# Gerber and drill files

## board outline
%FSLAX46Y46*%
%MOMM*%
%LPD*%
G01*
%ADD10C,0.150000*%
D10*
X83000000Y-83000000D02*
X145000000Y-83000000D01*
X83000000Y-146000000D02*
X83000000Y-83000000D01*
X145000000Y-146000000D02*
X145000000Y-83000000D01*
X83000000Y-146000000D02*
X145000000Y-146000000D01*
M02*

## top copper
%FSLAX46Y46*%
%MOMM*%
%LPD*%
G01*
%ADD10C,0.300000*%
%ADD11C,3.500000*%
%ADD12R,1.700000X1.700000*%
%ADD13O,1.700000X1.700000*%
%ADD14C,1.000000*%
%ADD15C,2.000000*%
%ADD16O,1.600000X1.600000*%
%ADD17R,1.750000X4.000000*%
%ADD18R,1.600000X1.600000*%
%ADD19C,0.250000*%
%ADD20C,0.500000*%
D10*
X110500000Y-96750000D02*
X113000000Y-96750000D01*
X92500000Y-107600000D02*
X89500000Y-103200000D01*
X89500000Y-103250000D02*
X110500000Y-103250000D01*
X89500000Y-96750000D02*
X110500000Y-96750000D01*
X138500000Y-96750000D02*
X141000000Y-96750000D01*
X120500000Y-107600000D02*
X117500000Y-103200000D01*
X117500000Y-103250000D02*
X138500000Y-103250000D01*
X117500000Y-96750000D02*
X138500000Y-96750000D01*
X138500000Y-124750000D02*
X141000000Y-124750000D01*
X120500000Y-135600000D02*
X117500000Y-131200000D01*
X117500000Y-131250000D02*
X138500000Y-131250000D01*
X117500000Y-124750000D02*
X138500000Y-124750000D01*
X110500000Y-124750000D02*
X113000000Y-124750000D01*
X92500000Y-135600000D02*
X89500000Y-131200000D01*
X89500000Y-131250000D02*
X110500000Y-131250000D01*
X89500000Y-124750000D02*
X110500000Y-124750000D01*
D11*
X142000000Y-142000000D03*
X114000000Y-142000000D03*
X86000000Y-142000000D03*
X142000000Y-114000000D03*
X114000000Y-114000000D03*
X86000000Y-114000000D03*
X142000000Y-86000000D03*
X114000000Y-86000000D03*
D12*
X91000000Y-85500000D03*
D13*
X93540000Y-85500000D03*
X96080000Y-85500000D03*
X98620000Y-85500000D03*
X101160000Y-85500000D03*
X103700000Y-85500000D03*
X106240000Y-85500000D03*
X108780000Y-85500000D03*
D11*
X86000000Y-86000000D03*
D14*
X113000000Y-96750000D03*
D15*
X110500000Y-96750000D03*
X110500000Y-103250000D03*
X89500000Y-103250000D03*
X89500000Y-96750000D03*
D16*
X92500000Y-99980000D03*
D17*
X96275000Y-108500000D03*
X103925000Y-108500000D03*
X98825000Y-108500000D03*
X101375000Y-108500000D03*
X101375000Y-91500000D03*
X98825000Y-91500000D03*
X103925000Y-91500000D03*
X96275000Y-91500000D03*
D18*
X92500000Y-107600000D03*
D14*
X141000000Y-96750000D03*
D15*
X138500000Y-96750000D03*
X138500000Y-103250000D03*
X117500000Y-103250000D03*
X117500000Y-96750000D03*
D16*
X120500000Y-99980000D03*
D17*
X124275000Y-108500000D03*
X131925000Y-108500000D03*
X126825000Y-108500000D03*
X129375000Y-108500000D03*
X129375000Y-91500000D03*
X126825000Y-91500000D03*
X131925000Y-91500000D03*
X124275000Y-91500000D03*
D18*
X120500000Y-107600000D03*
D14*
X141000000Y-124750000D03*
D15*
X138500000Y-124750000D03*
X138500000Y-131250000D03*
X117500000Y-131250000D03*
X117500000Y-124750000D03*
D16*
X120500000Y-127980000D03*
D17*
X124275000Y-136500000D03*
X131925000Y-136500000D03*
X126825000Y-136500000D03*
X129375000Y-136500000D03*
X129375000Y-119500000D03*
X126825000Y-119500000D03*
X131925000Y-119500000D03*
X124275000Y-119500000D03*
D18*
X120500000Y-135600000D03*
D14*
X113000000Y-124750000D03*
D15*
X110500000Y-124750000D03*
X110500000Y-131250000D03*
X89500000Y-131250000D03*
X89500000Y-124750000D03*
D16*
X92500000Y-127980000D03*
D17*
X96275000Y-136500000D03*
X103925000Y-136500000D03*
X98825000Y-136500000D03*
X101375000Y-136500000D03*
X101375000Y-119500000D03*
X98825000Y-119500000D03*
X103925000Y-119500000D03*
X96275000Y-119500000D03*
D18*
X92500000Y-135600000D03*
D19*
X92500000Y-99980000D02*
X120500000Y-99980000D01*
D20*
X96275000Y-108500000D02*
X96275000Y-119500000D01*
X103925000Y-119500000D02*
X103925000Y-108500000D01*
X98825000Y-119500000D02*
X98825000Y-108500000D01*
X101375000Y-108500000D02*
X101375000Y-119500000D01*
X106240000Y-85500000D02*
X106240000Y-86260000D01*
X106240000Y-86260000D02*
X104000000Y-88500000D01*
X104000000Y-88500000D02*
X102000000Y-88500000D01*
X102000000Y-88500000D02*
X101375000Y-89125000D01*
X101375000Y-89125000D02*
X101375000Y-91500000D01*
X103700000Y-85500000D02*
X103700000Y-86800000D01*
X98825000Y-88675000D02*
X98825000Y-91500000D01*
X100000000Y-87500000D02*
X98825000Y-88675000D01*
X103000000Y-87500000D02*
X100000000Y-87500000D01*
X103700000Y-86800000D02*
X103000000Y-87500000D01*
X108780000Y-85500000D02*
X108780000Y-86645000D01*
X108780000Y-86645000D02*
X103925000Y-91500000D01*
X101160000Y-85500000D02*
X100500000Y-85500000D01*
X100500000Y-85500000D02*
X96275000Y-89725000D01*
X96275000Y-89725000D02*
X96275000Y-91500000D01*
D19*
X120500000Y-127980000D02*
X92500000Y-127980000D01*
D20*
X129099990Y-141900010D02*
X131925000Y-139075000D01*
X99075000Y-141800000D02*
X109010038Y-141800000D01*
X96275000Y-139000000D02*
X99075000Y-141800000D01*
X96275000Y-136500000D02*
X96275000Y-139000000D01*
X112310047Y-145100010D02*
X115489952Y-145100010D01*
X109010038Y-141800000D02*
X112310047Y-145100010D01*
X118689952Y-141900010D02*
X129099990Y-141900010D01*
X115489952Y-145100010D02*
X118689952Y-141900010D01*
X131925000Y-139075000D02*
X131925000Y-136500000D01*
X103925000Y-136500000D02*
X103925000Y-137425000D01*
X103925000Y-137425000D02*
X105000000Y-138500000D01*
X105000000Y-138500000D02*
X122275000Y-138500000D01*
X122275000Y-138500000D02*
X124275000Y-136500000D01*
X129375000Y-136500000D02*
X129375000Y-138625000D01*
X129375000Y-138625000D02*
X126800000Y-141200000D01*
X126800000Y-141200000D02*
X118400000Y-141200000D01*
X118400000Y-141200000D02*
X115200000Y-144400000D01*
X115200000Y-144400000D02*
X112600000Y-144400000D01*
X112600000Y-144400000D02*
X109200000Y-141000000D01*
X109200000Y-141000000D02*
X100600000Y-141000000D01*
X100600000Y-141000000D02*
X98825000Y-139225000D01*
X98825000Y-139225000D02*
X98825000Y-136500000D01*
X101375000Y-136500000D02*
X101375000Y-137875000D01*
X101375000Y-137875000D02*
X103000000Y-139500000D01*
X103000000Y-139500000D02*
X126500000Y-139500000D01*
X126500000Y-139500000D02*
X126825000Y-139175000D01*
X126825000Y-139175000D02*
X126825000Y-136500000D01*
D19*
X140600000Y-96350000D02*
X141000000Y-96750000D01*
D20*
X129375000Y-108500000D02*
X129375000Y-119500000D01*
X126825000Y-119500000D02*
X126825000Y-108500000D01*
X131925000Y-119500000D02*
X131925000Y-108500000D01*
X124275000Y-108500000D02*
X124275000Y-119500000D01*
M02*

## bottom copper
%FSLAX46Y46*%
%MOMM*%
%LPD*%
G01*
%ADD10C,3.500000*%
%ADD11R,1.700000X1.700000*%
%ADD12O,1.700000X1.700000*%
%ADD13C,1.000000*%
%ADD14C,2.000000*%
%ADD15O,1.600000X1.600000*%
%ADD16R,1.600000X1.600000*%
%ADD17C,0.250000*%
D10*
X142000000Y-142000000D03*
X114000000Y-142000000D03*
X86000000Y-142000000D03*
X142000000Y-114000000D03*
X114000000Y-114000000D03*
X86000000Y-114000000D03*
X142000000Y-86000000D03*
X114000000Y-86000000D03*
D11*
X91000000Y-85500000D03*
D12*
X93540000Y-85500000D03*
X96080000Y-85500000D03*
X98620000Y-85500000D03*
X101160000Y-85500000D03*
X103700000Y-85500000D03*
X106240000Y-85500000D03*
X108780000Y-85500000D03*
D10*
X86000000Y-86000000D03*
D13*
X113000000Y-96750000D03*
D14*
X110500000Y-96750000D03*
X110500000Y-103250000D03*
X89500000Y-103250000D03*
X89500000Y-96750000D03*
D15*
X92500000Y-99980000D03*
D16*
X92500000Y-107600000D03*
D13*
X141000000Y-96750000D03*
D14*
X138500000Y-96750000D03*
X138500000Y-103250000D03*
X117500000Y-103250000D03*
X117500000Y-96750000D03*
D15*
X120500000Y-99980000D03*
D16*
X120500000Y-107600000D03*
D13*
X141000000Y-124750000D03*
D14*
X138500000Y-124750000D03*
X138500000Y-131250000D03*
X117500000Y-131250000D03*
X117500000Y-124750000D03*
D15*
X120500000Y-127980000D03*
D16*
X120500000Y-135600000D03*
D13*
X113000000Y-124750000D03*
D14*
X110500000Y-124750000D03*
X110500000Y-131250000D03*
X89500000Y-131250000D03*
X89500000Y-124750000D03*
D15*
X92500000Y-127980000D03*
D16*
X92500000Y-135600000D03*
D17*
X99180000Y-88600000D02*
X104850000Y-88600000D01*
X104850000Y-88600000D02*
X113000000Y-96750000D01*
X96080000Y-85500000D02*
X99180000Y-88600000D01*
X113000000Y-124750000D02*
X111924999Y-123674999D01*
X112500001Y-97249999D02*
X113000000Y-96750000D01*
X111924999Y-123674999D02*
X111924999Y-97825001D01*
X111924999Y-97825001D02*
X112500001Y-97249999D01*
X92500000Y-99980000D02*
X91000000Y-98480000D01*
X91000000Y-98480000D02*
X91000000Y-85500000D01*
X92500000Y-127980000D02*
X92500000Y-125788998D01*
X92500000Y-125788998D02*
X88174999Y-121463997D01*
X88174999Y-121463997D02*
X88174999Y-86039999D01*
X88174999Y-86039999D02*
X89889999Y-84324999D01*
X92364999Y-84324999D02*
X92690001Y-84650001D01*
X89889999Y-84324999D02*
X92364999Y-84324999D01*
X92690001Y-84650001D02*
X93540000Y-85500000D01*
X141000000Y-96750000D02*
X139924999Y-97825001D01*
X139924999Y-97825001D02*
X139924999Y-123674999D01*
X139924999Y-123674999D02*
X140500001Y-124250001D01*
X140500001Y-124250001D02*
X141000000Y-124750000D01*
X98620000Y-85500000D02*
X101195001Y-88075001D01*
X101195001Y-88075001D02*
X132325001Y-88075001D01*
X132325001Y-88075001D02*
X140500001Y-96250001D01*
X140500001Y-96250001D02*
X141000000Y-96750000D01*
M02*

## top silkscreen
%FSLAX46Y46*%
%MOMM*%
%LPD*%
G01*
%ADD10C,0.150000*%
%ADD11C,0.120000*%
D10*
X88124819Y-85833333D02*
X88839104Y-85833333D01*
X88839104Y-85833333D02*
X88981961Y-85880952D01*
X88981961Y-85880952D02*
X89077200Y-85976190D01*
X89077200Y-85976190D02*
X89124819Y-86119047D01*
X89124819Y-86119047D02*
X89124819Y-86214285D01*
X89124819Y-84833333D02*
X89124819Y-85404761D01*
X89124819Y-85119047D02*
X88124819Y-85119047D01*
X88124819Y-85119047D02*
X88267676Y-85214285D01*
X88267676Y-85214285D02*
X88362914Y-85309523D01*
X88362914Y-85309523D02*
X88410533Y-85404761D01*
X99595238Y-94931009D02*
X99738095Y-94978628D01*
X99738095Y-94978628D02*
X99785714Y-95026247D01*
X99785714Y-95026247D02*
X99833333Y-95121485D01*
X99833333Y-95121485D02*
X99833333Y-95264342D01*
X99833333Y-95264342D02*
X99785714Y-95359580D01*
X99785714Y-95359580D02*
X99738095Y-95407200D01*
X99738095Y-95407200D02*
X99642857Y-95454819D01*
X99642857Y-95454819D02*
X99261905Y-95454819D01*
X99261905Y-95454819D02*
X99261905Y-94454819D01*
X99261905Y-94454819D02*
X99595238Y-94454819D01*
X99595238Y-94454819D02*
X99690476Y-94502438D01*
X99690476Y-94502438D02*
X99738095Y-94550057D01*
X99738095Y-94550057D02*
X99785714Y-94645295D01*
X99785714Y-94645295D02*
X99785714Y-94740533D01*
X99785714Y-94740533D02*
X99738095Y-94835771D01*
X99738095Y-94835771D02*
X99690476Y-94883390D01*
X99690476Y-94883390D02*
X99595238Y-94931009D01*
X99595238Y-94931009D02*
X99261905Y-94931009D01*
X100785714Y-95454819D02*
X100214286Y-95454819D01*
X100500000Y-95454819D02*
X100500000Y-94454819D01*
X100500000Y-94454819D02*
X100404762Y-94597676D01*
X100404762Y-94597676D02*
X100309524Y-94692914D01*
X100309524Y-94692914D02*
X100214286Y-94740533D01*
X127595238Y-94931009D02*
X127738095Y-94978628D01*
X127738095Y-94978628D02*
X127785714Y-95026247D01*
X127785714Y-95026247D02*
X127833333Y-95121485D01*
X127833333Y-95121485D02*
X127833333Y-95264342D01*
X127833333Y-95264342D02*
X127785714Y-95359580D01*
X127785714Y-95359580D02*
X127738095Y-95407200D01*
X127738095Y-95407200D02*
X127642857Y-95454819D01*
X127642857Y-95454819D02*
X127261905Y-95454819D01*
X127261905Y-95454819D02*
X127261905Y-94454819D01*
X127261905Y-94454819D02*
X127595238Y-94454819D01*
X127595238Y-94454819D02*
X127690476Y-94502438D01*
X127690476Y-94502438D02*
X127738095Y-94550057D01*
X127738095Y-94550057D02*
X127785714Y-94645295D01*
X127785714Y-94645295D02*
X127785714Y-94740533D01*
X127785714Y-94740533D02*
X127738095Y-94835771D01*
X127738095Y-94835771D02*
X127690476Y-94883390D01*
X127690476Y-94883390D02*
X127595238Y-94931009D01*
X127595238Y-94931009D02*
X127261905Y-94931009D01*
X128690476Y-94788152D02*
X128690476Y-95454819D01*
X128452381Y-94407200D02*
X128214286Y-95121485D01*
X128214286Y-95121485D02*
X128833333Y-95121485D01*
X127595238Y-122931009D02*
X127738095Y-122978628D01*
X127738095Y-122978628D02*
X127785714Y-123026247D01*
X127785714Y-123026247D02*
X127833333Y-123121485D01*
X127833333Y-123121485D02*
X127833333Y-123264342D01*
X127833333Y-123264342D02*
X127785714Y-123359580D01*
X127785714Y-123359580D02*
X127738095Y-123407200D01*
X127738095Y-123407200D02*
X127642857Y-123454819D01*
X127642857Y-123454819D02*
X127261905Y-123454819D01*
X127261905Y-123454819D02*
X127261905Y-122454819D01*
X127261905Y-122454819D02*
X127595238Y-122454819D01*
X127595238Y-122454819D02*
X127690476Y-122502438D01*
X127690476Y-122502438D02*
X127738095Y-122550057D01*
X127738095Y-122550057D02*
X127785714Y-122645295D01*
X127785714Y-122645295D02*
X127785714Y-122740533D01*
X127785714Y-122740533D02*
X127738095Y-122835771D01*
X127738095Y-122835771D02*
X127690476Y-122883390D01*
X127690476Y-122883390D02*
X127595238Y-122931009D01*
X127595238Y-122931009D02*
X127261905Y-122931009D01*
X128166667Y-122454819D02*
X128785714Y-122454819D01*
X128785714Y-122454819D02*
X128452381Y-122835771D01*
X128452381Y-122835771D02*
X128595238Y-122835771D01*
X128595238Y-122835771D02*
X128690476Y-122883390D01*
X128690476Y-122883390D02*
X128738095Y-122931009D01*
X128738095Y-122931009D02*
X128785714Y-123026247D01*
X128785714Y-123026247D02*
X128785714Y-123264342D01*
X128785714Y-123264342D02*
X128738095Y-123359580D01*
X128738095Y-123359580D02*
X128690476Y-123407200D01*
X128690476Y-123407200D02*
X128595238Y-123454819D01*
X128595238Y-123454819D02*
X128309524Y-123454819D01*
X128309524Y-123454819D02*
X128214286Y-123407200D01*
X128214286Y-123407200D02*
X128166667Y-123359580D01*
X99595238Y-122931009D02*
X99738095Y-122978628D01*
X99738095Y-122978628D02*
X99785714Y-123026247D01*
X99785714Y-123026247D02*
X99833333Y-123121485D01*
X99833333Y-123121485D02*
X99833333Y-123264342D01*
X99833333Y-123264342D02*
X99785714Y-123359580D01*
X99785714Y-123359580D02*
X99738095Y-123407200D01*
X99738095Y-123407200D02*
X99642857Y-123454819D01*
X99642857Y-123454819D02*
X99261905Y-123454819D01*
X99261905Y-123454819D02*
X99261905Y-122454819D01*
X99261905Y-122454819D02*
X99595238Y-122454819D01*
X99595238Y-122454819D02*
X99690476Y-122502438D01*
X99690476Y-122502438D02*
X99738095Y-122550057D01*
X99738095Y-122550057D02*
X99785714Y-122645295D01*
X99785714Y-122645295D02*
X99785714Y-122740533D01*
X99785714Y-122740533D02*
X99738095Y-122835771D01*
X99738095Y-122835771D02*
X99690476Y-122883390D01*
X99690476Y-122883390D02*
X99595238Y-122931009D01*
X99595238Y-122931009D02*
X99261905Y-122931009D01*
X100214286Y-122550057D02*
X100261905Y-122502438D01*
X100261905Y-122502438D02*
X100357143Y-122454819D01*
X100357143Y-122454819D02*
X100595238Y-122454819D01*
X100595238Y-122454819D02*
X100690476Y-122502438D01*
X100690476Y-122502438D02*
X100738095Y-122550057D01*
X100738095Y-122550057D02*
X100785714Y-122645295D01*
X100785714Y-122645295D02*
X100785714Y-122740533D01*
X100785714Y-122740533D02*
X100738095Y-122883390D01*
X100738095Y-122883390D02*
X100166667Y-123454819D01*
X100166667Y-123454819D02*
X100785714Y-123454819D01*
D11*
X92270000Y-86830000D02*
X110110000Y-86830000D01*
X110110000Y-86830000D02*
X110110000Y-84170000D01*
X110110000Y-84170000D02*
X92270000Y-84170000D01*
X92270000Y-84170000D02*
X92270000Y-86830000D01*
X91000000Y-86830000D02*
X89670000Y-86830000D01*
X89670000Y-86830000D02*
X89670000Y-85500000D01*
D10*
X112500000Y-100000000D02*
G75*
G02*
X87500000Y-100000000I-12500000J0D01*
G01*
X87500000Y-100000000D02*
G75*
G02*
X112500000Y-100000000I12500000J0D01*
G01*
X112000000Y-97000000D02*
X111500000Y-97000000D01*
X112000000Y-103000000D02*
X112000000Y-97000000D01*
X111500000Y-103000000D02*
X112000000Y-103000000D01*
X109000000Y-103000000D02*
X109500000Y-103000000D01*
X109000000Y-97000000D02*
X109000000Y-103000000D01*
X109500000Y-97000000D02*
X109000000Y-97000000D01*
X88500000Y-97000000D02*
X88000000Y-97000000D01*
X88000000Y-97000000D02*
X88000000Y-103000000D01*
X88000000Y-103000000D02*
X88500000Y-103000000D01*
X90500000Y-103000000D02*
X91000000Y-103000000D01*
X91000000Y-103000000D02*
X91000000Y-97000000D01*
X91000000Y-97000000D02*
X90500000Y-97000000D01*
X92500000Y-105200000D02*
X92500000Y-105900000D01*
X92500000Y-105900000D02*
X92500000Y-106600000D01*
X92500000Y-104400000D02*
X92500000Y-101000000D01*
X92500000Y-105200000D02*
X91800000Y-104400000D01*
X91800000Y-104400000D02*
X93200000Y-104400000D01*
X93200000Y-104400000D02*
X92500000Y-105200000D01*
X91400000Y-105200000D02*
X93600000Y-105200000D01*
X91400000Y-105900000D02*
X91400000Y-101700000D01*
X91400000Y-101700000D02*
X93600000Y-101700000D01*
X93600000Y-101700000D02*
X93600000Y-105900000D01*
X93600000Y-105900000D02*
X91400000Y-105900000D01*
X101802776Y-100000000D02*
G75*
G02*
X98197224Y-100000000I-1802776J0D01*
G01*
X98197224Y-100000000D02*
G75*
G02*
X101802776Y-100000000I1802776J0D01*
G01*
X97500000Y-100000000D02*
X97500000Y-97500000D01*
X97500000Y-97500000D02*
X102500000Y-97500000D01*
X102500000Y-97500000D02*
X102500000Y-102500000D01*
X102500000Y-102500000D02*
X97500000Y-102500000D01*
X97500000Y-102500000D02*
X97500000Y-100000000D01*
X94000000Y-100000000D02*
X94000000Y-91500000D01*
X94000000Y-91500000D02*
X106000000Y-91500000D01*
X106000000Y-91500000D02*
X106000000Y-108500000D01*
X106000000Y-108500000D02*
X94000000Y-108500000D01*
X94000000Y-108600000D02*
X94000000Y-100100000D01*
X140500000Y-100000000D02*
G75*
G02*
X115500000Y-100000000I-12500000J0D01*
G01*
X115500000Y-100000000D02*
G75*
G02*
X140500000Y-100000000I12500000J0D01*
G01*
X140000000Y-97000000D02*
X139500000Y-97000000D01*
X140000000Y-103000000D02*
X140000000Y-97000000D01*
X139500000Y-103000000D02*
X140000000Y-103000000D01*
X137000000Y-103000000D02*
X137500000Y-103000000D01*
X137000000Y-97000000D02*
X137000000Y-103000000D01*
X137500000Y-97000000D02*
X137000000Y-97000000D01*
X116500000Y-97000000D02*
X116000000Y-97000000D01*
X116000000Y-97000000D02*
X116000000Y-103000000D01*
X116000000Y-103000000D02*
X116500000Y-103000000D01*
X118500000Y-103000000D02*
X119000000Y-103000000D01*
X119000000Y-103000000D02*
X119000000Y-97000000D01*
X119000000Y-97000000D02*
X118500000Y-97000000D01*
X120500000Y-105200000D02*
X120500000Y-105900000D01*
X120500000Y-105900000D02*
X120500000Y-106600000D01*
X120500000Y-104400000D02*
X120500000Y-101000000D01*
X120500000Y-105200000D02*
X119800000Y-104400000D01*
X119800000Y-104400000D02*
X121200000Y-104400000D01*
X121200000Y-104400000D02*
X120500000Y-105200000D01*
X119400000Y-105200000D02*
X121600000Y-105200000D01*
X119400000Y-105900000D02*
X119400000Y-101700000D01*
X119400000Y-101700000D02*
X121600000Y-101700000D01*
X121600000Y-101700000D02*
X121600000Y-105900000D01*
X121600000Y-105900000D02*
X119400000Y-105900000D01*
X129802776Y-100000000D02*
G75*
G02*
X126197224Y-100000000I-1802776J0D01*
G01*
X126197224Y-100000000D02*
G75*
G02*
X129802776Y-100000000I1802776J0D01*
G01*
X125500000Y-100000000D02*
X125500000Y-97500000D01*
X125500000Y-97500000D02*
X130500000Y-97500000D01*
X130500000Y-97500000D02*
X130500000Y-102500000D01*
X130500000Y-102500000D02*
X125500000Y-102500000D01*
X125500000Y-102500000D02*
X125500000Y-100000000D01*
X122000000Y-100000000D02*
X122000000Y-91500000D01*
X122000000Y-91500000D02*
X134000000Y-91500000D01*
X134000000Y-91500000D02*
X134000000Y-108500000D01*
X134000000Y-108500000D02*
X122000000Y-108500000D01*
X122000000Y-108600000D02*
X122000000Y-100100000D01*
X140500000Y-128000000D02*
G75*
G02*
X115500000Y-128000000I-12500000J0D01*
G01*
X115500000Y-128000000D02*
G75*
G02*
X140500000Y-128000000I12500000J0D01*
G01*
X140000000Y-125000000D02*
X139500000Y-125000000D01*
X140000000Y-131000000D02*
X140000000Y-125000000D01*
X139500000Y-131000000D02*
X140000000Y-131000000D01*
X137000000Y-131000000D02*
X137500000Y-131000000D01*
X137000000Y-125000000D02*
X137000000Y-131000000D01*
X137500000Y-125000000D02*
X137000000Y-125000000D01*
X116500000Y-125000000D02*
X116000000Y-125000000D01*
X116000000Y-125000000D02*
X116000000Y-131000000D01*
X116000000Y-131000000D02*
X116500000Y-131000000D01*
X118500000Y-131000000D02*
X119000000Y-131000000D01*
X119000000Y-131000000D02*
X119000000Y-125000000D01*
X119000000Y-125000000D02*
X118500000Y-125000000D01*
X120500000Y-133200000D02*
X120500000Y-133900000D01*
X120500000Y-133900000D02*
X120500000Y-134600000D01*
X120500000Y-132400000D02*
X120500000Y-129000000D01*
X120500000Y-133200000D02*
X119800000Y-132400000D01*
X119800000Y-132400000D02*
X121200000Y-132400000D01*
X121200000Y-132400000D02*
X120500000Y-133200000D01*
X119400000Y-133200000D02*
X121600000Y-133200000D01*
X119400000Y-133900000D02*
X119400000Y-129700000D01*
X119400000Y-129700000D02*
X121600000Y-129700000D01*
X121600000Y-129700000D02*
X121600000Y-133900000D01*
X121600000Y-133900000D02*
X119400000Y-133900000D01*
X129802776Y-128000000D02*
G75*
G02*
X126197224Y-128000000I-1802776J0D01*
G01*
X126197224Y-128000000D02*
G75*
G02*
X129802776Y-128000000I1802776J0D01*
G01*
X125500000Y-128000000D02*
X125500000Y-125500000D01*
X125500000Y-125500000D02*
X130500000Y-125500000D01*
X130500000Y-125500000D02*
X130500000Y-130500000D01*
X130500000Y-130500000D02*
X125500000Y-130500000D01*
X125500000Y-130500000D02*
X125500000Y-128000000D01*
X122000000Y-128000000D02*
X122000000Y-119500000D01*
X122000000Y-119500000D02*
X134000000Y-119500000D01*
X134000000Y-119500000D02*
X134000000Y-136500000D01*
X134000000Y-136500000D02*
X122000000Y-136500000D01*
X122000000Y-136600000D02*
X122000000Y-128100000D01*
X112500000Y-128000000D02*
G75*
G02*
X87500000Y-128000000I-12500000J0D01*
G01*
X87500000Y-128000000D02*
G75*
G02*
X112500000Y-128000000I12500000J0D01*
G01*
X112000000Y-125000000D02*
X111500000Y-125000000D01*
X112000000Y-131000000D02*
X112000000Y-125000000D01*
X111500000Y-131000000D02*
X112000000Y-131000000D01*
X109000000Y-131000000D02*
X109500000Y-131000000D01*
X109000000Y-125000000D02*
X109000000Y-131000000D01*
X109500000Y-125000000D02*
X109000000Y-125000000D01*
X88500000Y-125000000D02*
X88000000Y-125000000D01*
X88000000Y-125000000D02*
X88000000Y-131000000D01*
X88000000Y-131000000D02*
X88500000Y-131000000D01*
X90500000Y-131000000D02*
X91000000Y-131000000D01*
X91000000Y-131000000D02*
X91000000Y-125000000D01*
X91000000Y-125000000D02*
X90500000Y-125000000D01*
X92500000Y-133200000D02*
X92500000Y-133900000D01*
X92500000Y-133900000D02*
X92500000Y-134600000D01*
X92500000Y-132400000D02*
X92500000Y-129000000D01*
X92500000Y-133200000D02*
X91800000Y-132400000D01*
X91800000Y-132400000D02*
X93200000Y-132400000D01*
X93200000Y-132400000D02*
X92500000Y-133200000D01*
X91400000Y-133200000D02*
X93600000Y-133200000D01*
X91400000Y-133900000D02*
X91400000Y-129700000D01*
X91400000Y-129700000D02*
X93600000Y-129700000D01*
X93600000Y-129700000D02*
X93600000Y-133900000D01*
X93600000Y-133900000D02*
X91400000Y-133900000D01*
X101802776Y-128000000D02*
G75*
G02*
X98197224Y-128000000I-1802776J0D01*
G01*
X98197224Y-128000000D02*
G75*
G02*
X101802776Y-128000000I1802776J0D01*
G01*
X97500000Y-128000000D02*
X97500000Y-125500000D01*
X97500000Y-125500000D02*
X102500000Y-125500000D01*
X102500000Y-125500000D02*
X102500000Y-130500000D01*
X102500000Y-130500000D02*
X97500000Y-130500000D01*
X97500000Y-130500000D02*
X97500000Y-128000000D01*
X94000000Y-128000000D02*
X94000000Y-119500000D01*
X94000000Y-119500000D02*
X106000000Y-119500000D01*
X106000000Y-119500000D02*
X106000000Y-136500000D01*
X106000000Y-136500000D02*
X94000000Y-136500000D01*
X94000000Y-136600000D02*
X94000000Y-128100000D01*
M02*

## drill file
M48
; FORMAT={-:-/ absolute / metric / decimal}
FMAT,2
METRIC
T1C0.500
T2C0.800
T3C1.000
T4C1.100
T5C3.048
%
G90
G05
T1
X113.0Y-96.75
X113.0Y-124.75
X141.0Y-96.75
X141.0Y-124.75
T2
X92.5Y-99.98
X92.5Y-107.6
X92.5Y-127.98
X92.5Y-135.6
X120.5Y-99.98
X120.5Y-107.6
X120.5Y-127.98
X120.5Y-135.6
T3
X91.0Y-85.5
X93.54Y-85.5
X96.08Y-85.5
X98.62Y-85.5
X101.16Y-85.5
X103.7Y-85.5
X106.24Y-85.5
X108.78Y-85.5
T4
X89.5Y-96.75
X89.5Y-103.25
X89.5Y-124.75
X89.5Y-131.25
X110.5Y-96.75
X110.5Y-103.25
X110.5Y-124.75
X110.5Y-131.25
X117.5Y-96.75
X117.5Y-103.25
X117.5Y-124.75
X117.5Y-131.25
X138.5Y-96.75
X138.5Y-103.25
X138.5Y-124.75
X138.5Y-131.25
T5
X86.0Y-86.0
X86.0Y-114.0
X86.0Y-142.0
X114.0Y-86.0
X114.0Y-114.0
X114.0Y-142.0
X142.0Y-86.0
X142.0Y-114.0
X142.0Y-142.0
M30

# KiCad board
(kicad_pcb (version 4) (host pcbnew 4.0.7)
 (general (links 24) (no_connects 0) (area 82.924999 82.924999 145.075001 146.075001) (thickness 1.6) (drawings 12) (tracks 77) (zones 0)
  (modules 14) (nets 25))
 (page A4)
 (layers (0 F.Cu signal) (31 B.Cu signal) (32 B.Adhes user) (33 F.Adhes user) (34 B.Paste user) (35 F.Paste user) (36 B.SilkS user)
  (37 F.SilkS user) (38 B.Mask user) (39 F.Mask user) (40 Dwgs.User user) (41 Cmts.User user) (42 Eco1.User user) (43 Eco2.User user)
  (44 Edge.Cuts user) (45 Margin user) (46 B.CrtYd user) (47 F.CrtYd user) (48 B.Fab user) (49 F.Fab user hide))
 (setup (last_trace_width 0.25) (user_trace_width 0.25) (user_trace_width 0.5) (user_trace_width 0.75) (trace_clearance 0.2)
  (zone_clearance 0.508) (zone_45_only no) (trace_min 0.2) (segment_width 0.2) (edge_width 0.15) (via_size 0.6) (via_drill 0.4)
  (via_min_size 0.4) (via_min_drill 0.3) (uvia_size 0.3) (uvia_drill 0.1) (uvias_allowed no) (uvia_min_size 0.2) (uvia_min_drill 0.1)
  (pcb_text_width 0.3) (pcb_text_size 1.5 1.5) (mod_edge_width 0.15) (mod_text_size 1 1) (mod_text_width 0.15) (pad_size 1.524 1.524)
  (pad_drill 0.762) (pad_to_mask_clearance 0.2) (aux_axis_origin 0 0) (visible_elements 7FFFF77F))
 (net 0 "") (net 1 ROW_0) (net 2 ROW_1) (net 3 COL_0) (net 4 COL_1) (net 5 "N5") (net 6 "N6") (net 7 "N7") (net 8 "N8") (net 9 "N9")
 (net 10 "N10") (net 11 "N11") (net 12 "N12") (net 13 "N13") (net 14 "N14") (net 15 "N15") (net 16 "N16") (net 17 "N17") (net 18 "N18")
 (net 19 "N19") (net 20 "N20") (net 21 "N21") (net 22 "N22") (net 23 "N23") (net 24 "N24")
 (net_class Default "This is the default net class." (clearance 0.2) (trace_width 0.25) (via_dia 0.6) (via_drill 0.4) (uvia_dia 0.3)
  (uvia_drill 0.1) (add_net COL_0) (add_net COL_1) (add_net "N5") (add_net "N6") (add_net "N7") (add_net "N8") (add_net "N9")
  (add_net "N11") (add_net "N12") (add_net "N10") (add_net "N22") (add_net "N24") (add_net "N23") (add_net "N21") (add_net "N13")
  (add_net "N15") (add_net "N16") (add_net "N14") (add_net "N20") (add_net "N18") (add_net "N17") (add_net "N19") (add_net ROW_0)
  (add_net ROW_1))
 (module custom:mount (layer F.Cu) (at 142 142)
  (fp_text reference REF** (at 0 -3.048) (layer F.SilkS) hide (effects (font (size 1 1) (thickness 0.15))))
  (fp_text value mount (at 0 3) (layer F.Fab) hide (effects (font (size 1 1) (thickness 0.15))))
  (pad 0 thru_hole circle (at 0 0) (size 3.5 3.5) (drill 3.048) (layers *.Cu *.Mask)))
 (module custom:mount (layer F.Cu) (at 114 142)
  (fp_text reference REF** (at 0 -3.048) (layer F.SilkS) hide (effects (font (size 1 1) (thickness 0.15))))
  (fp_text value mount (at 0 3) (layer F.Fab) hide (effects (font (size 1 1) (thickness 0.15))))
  (pad 0 thru_hole circle (at 0 0) (size 3.5 3.5) (drill 3.048) (layers *.Cu *.Mask)))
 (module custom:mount (layer F.Cu) (at 86 142)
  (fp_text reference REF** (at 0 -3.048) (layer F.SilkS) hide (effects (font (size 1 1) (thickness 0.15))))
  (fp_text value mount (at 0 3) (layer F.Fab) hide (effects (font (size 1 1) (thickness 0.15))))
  (pad 0 thru_hole circle (at 0 0) (size 3.5 3.5) (drill 3.048) (layers *.Cu *.Mask)))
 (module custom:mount (layer F.Cu) (at 142 114)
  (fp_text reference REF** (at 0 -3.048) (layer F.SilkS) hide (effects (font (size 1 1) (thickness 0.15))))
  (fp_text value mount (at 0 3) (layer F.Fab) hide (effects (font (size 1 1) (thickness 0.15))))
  (pad 0 thru_hole circle (at 0 0) (size 3.5 3.5) (drill 3.048) (layers *.Cu *.Mask)))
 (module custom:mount (layer F.Cu) (at 114 114)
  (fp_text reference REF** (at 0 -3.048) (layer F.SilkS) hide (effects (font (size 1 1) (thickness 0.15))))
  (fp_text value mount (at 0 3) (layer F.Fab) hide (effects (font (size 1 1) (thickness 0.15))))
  (pad 0 thru_hole circle (at 0 0) (size 3.5 3.5) (drill 3.048) (layers *.Cu *.Mask)))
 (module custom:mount (layer F.Cu) (at 86 114)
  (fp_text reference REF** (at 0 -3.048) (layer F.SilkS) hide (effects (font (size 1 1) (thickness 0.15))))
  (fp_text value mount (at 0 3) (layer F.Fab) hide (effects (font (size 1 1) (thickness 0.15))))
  (pad 0 thru_hole circle (at 0 0) (size 3.5 3.5) (drill 3.048) (layers *.Cu *.Mask)))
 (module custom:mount (layer F.Cu) (at 142 86)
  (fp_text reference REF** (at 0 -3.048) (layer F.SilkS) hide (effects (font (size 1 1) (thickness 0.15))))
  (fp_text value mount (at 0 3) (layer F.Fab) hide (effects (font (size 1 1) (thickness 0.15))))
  (pad 0 thru_hole circle (at 0 0) (size 3.5 3.5) (drill 3.048) (layers *.Cu *.Mask)))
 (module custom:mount (layer F.Cu) (at 114 86)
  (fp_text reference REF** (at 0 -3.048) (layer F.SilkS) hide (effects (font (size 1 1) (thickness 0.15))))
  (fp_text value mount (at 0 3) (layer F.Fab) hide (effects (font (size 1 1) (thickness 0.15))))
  (pad 0 thru_hole circle (at 0 0) (size 3.5 3.5) (drill 3.048) (layers *.Cu *.Mask)))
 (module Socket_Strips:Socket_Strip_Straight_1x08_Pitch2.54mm (layer F.Cu) (at 91 85.5 90)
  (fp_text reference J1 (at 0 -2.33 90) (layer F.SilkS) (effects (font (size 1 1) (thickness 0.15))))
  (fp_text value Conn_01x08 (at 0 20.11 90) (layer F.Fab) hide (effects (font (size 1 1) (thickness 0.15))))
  (fp_line (start -1.33 1.27) (end -1.33 19.11) (layer F.SilkS) (width 0.12))
  (fp_line (start -1.33 19.11) (end 1.33 19.11) (layer F.SilkS) (width 0.12))
  (fp_line (start 1.33 19.11) (end 1.33 1.27) (layer F.SilkS) (width 0.12))
  (fp_line (start 1.33 1.27) (end -1.33 1.27) (layer F.SilkS) (width 0.12))
  (fp_line (start -1.33 0) (end -1.33 -1.33) (layer F.SilkS) (width 0.12))
  (fp_line (start -1.33 -1.33) (end 0 -1.33) (layer F.SilkS) (width 0.12))
  (pad 1 thru_hole rect (at 0 0 90) (size 1.7 1.7) (drill 1) (layers *.Cu *.Mask) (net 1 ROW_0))
  (pad 2 thru_hole oval (at 0 2.54 90) (size 1.7 1.7) (drill 1) (layers *.Cu *.Mask) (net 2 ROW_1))
  (pad 3 thru_hole oval (at 0 5.08 90) (size 1.7 1.7) (drill 1) (layers *.Cu *.Mask) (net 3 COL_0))
  (pad 4 thru_hole oval (at 0 7.62 90) (size 1.7 1.7) (drill 1) (layers *.Cu *.Mask) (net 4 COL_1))
  (pad 5 thru_hole oval (at 0 10.16 90) (size 1.7 1.7) (drill 1) (layers *.Cu *.Mask) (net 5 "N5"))
  (pad 6 thru_hole oval (at 0 12.7 90) (size 1.7 1.7) (drill 1) (layers *.Cu *.Mask) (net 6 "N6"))
  (pad 7 thru_hole oval (at 0 15.24 90) (size 1.7 1.7) (drill 1) (layers *.Cu *.Mask) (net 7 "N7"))
  (pad 8 thru_hole oval (at 0 17.78 90) (size 1.7 1.7) (drill 1) (layers *.Cu *.Mask) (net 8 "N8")))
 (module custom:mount (layer F.Cu) (at 86 86)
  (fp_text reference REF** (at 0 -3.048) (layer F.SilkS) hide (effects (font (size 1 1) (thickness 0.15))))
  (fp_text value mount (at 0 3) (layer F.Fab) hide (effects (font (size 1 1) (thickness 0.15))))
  (pad 0 thru_hole circle (at 0 0) (size 3.5 3.5) (drill 3.048) (layers *.Cu *.Mask)))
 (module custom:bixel (layer F.Cu) (at 100 100)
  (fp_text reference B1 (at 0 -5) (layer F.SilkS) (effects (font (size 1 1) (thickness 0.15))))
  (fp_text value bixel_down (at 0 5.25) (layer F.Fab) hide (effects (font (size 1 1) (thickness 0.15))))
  (fp_line (start 10.5 -3.25) (end 13 -3.25) (layer F.Cu) (width 0.3))
  (fp_line (start -7.5 7.6) (end -10.5 3.2) (layer F.Cu) (width 0.3))
  (fp_line (start -10.5 3.25) (end 10.5 3.25) (layer F.Cu) (width 0.3))
  (fp_line (start -10.5 -3.25) (end 10.5 -3.25) (layer F.Cu) (width 0.3))
  (fp_circle (center 0 0) (end 0 12.5) (layer F.SilkS) (width 0.15))
  (fp_line (start 12 -3) (end 11.5 -3) (layer F.SilkS) (width 0.15))
  (fp_line (start 12 3) (end 12 -3) (layer F.SilkS) (width 0.15))
  (fp_line (start 11.5 3) (end 12 3) (layer F.SilkS) (width 0.15))
  (fp_line (start 9 3) (end 9.5 3) (layer F.SilkS) (width 0.15))
  (fp_line (start 9 -3) (end 9 3) (layer F.SilkS) (width 0.15))
  (fp_line (start 9.5 -3) (end 9 -3) (layer F.SilkS) (width 0.15))
  (fp_line (start -11.5 -3) (end -12 -3) (layer F.SilkS) (width 0.15))
  (fp_line (start -12 -3) (end -12 3) (layer F.SilkS) (width 0.15))
  (fp_line (start -12 3) (end -11.5 3) (layer F.SilkS) (width 0.15))
  (fp_line (start -9.5 3) (end -9 3) (layer F.SilkS) (width 0.15))
  (fp_line (start -9 3) (end -9 -3) (layer F.SilkS) (width 0.15))
  (fp_line (start -9 -3) (end -9.5 -3) (layer F.SilkS) (width 0.15))
  (fp_line (start -7.5 5.2) (end -7.5 5.9) (layer F.SilkS) (width 0.15))
  (fp_line (start -7.5 5.9) (end -7.5 6.6) (layer F.SilkS) (width 0.15))
  (fp_line (start -7.5 4.4) (end -7.5 1) (layer F.SilkS) (width 0.15))
  (fp_line (start -7.5 5.2) (end -8.2 4.4) (layer F.SilkS) (width 0.15))
  (fp_line (start -8.2 4.4) (end -6.8 4.4) (layer F.SilkS) (width 0.15))
  (fp_line (start -6.8 4.4) (end -7.5 5.2) (layer F.SilkS) (width 0.15))
  (fp_line (start -8.6 5.2) (end -6.4 5.2) (layer F.SilkS) (width 0.15))
  (fp_line (start -8.6 5.9) (end -8.6 1.7) (layer F.SilkS) (width 0.15))
  (fp_line (start -8.6 1.7) (end -6.4 1.7) (layer F.SilkS) (width 0.15))
  (fp_line (start -6.4 1.7) (end -6.4 5.9) (layer F.SilkS) (width 0.15))
  (fp_line (start -6.4 5.9) (end -8.6 5.9) (layer F.SilkS) (width 0.15))
  (fp_circle (center 0 0) (end 1 1.5) (layer F.SilkS) (width 0.15))
  (fp_line (start -2.5 0) (end -2.5 -2.5) (layer F.SilkS) (width 0.15))
  (fp_line (start -2.5 -2.5) (end 2.5 -2.5) (layer F.SilkS) (width 0.15))
  (fp_line (start 2.5 -2.5) (end 2.5 2.5) (layer F.SilkS) (width 0.15))
  (fp_line (start 2.5 2.5) (end -2.5 2.5) (layer F.SilkS) (width 0.15))
  (fp_line (start -2.5 2.5) (end -2.5 0) (layer F.SilkS) (width 0.15))
  (fp_line (start -6 0) (end -6 -8.5) (layer F.SilkS) (width 0.15))
  (fp_line (start -6 -8.5) (end 6 -8.5) (layer F.SilkS) (width 0.15))
  (fp_line (start 6 -8.5) (end 6 8.5) (layer F.SilkS) (width 0.15))
  (fp_line (start 6 8.5) (end -6 8.5) (layer F.SilkS) (width 0.15))
  (fp_line (start -6 8.6) (end -6 0.1) (layer F.SilkS) (width 0.15))
  (pad 10 thru_hole circle (at 13 -3.25) (size 1 1) (drill 0.5) (layers *.Cu *.Mask) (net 3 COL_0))
  (pad "" thru_hole circle (at 10.5 -3.25) (size 2 2) (drill 1.1) (layers *.Cu *.Mask))
  (pad "" thru_hole circle (at 10.5 3.25) (size 2 2) (drill 1.1) (layers *.Cu *.Mask))
  (pad "" thru_hole circle (at -10.5 3.25) (size 2 2) (drill 1.1) (layers *.Cu *.Mask))
  (pad "" thru_hole circle (at -10.5 -3.25) (size 2 2) (drill 1.1) (layers *.Cu *.Mask))
  (pad 9 thru_hole oval (at -7.5 -0.02 90) (size 1.6 1.6) (drill 0.8) (layers *.Cu *.Mask) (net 1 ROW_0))
  (pad 5 smd rect (at -3.725 8.5) (size 1.75 4) (layers F.Cu F.Paste F.Mask) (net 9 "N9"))
  (pad 8 smd rect (at 3.925 8.5) (size 1.75 4) (layers F.Cu F.Paste F.Mask) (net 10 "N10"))
  (pad 6 smd rect (at -1.175 8.5) (size 1.75 4) (layers F.Cu F.Paste F.Mask) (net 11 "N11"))
  (pad 7 smd rect (at 1.375 8.5) (size 1.75 4) (layers F.Cu F.Paste F.Mask) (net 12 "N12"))
  (pad 3 smd rect (at 1.375 -8.5) (size 1.75 4) (layers F.Cu F.Paste F.Mask) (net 7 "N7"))
  (pad 2 smd rect (at -1.175 -8.5) (size 1.75 4) (layers F.Cu F.Paste F.Mask) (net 6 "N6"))
  (pad 4 smd rect (at 3.925 -8.5) (size 1.75 4) (layers F.Cu F.Paste F.Mask) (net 8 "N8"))
  (pad 1 smd rect (at -3.725 -8.5) (size 1.75 4) (layers F.Cu F.Paste F.Mask) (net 5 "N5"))
  (pad "" thru_hole rect (at -7.5 7.6 90) (size 1.6 1.6) (drill 0.8) (layers *.Cu *.Mask)))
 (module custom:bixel (layer F.Cu) (at 128 100)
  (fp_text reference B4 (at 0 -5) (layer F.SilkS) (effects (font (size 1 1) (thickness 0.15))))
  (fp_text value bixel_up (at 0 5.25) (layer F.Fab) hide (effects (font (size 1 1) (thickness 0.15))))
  (fp_line (start 10.5 -3.25) (end 13 -3.25) (layer F.Cu) (width 0.3))
  (fp_line (start -7.5 7.6) (end -10.5 3.2) (layer F.Cu) (width 0.3))
  (fp_line (start -10.5 3.25) (end 10.5 3.25) (layer F.Cu) (width 0.3))
  (fp_line (start -10.5 -3.25) (end 10.5 -3.25) (layer F.Cu) (width 0.3))
  (fp_circle (center 0 0) (end 0 12.5) (layer F.SilkS) (width 0.15))
  (fp_line (start 12 -3) (end 11.5 -3) (layer F.SilkS) (width 0.15))
  (fp_line (start 12 3) (end 12 -3) (layer F.SilkS) (width 0.15))
  (fp_line (start 11.5 3) (end 12 3) (layer F.SilkS) (width 0.15))
  (fp_line (start 9 3) (end 9.5 3) (layer F.SilkS) (width 0.15))
  (fp_line (start 9 -3) (end 9 3) (layer F.SilkS) (width 0.15))
  (fp_line (start 9.5 -3) (end 9 -3) (layer F.SilkS) (width 0.15))
  (fp_line (start -11.5 -3) (end -12 -3) (layer F.SilkS) (width 0.15))
  (fp_line (start -12 -3) (end -12 3) (layer F.SilkS) (width 0.15))
  (fp_line (start -12 3) (end -11.5 3) (layer F.SilkS) (width 0.15))
  (fp_line (start -9.5 3) (end -9 3) (layer F.SilkS) (width 0.15))
  (fp_line (start -9 3) (end -9 -3) (layer F.SilkS) (width 0.15))
  (fp_line (start -9 -3) (end -9.5 -3) (layer F.SilkS) (width 0.15))
  (fp_line (start -7.5 5.2) (end -7.5 5.9) (layer F.SilkS) (width 0.15))
  (fp_line (start -7.5 5.9) (end -7.5 6.6) (layer F.SilkS) (width 0.15))
  (fp_line (start -7.5 4.4) (end -7.5 1) (layer F.SilkS) (width 0.15))
  (fp_line (start -7.5 5.2) (end -8.2 4.4) (layer F.SilkS) (width 0.15))
  (fp_line (start -8.2 4.4) (end -6.8 4.4) (layer F.SilkS) (width 0.15))
  (fp_line (start -6.8 4.4) (end -7.5 5.2) (layer F.SilkS) (width 0.15))
  (fp_line (start -8.6 5.2) (end -6.4 5.2) (layer F.SilkS) (width 0.15))
  (fp_line (start -8.6 5.9) (end -8.6 1.7) (layer F.SilkS) (width 0.15))
  (fp_line (start -8.6 1.7) (end -6.4 1.7) (layer F.SilkS) (width 0.15))
  (fp_line (start -6.4 1.7) (end -6.4 5.9) (layer F.SilkS) (width 0.15))
  (fp_line (start -6.4 5.9) (end -8.6 5.9) (layer F.SilkS) (width 0.15))
  (fp_circle (center 0 0) (end 1 1.5) (layer F.SilkS) (width 0.15))
  (fp_line (start -2.5 0) (end -2.5 -2.5) (layer F.SilkS) (width 0.15))
  (fp_line (start -2.5 -2.5) (end 2.5 -2.5) (layer F.SilkS) (width 0.15))
  (fp_line (start 2.5 -2.5) (end 2.5 2.5) (layer F.SilkS) (width 0.15))
  (fp_line (start 2.5 2.5) (end -2.5 2.5) (layer F.SilkS) (width 0.15))
  (fp_line (start -2.5 2.5) (end -2.5 0) (layer F.SilkS) (width 0.15))
  (fp_line (start -6 0) (end -6 -8.5) (layer F.SilkS) (width 0.15))
  (fp_line (start -6 -8.5) (end 6 -8.5) (layer F.SilkS) (width 0.15))
  (fp_line (start 6 -8.5) (end 6 8.5) (layer F.SilkS) (width 0.15))
  (fp_line (start 6 8.5) (end -6 8.5) (layer F.SilkS) (width 0.15))
  (fp_line (start -6 8.6) (end -6 0.1) (layer F.SilkS) (width 0.15))
  (pad 10 thru_hole circle (at 13 -3.25) (size 1 1) (drill 0.5) (layers *.Cu *.Mask) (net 4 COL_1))
  (pad "" thru_hole circle (at 10.5 -3.25) (size 2 2) (drill 1.1) (layers *.Cu *.Mask))
  (pad "" thru_hole circle (at 10.5 3.25) (size 2 2) (drill 1.1) (layers *.Cu *.Mask))
  (pad "" thru_hole circle (at -10.5 3.25) (size 2 2) (drill 1.1) (layers *.Cu *.Mask))
  (pad "" thru_hole circle (at -10.5 -3.25) (size 2 2) (drill 1.1) (layers *.Cu *.Mask))
  (pad 9 thru_hole oval (at -7.5 -0.02 90) (size 1.6 1.6) (drill 0.8) (layers *.Cu *.Mask) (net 1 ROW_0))
  (pad 5 smd rect (at -3.725 8.5) (size 1.75 4) (layers F.Cu F.Paste F.Mask) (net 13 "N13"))
  (pad 8 smd rect (at 3.925 8.5) (size 1.75 4) (layers F.Cu F.Paste F.Mask) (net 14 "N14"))
  (pad 6 smd rect (at -1.175 8.5) (size 1.75 4) (layers F.Cu F.Paste F.Mask) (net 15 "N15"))
  (pad 7 smd rect (at 1.375 8.5) (size 1.75 4) (layers F.Cu F.Paste F.Mask) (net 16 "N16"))
  (pad 3 smd rect (at 1.375 -8.5) (size 1.75 4) (layers F.Cu F.Paste F.Mask) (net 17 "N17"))
  (pad 2 smd rect (at -1.175 -8.5) (size 1.75 4) (layers F.Cu F.Paste F.Mask) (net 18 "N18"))
  (pad 4 smd rect (at 3.925 -8.5) (size 1.75 4) (layers F.Cu F.Paste F.Mask) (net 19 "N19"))
  (pad 1 smd rect (at -3.725 -8.5) (size 1.75 4) (layers F.Cu F.Paste F.Mask) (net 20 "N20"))
  (pad "" thru_hole rect (at -7.5 7.6 90) (size 1.6 1.6) (drill 0.8) (layers *.Cu *.Mask)))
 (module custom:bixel (layer F.Cu) (at 128 128)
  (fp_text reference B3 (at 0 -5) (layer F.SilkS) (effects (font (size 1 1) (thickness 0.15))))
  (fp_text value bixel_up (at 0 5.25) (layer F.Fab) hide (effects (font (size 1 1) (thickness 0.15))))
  (fp_line (start 10.5 -3.25) (end 13 -3.25) (layer F.Cu) (width 0.3))
  (fp_line (start -7.5 7.6) (end -10.5 3.2) (layer F.Cu) (width 0.3))
  (fp_line (start -10.5 3.25) (end 10.5 3.25) (layer F.Cu) (width 0.3))
  (fp_line (start -10.5 -3.25) (end 10.5 -3.25) (layer F.Cu) (width 0.3))
  (fp_circle (center 0 0) (end 0 12.5) (layer F.SilkS) (width 0.15))
  (fp_line (start 12 -3) (end 11.5 -3) (layer F.SilkS) (width 0.15))
  (fp_line (start 12 3) (end 12 -3) (layer F.SilkS) (width 0.15))
  (fp_line (start 11.5 3) (end 12 3) (layer F.SilkS) (width 0.15))
  (fp_line (start 9 3) (end 9.5 3) (layer F.SilkS) (width 0.15))
  (fp_line (start 9 -3) (end 9 3) (layer F.SilkS) (width 0.15))
  (fp_line (start 9.5 -3) (end 9 -3) (layer F.SilkS) (width 0.15))
  (fp_line (start -11.5 -3) (end -12 -3) (layer F.SilkS) (width 0.15))
  (fp_line (start -12 -3) (end -12 3) (layer F.SilkS) (width 0.15))
  (fp_line (start -12 3) (end -11.5 3) (layer F.SilkS) (width 0.15))
  (fp_line (start -9.5 3) (end -9 3) (layer F.SilkS) (width 0.15))
  (fp_line (start -9 3) (end -9 -3) (layer F.SilkS) (width 0.15))
  (fp_line (start -9 -3) (end -9.5 -3) (layer F.SilkS) (width 0.15))
  (fp_line (start -7.5 5.2) (end -7.5 5.9) (layer F.SilkS) (width 0.15))
  (fp_line (start -7.5 5.9) (end -7.5 6.6) (layer F.SilkS) (width 0.15))
  (fp_line (start -7.5 4.4) (end -7.5 1) (layer F.SilkS) (width 0.15))
  (fp_line (start -7.5 5.2) (end -8.2 4.4) (layer F.SilkS) (width 0.15))
  (fp_line (start -8.2 4.4) (end -6.8 4.4) (layer F.SilkS) (width 0.15))
  (fp_line (start -6.8 4.4) (end -7.5 5.2) (layer F.SilkS) (width 0.15))
  (fp_line (start -8.6 5.2) (end -6.4 5.2) (layer F.SilkS) (width 0.15))
  (fp_line (start -8.6 5.9) (end -8.6 1.7) (layer F.SilkS) (width 0.15))
  (fp_line (start -8.6 1.7) (end -6.4 1.7) (layer F.SilkS) (width 0.15))
  (fp_line (start -6.4 1.7) (end -6.4 5.9) (layer F.SilkS) (width 0.15))
  (fp_line (start -6.4 5.9) (end -8.6 5.9) (layer F.SilkS) (width 0.15))
  (fp_circle (center 0 0) (end 1 1.5) (layer F.SilkS) (width 0.15))
  (fp_line (start -2.5 0) (end -2.5 -2.5) (layer F.SilkS) (width 0.15))
  (fp_line (start -2.5 -2.5) (end 2.5 -2.5) (layer F.SilkS) (width 0.15))
  (fp_line (start 2.5 -2.5) (end 2.5 2.5) (layer F.SilkS) (width 0.15))
  (fp_line (start 2.5 2.5) (end -2.5 2.5) (layer F.SilkS) (width 0.15))
  (fp_line (start -2.5 2.5) (end -2.5 0) (layer F.SilkS) (width 0.15))
  (fp_line (start -6 0) (end -6 -8.5) (layer F.SilkS) (width 0.15))
  (fp_line (start -6 -8.5) (end 6 -8.5) (layer F.SilkS) (width 0.15))
  (fp_line (start 6 -8.5) (end 6 8.5) (layer F.SilkS) (width 0.15))
  (fp_line (start 6 8.5) (end -6 8.5) (layer F.SilkS) (width 0.15))
  (fp_line (start -6 8.6) (end -6 0.1) (layer F.SilkS) (width 0.15))
  (pad 10 thru_hole circle (at 13 -3.25) (size 1 1) (drill 0.5) (layers *.Cu *.Mask) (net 4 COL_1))
  (pad "" thru_hole circle (at 10.5 -3.25) (size 2 2) (drill 1.1) (layers *.Cu *.Mask))
  (pad "" thru_hole circle (at 10.5 3.25) (size 2 2) (drill 1.1) (layers *.Cu *.Mask))
  (pad "" thru_hole circle (at -10.5 3.25) (size 2 2) (drill 1.1) (layers *.Cu *.Mask))
  (pad "" thru_hole circle (at -10.5 -3.25) (size 2 2) (drill 1.1) (layers *.Cu *.Mask))
  (pad 9 thru_hole oval (at -7.5 -0.02 90) (size 1.6 1.6) (drill 0.8) (layers *.Cu *.Mask) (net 2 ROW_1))
  (pad 5 smd rect (at -3.725 8.5) (size 1.75 4) (layers F.Cu F.Paste F.Mask) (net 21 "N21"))
  (pad 8 smd rect (at 3.925 8.5) (size 1.75 4) (layers F.Cu F.Paste F.Mask) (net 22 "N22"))
  (pad 6 smd rect (at -1.175 8.5) (size 1.75 4) (layers F.Cu F.Paste F.Mask) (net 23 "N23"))
  (pad 7 smd rect (at 1.375 8.5) (size 1.75 4) (layers F.Cu F.Paste F.Mask) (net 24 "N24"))
  (pad 3 smd rect (at 1.375 -8.5) (size 1.75 4) (layers F.Cu F.Paste F.Mask) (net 16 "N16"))
  (pad 2 smd rect (at -1.175 -8.5) (size 1.75 4) (layers F.Cu F.Paste F.Mask) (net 15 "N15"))
  (pad 4 smd rect (at 3.925 -8.5) (size 1.75 4) (layers F.Cu F.Paste F.Mask) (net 14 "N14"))
  (pad 1 smd rect (at -3.725 -8.5) (size 1.75 4) (layers F.Cu F.Paste F.Mask) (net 13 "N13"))
  (pad "" thru_hole rect (at -7.5 7.6 90) (size 1.6 1.6) (drill 0.8) (layers *.Cu *.Mask)))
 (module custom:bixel (layer F.Cu) (at 100 128)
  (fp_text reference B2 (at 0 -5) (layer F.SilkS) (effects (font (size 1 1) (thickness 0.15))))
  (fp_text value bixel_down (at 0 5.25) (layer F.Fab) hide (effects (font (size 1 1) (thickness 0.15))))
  (fp_line (start 10.5 -3.25) (end 13 -3.25) (layer F.Cu) (width 0.3))
  (fp_line (start -7.5 7.6) (end -10.5 3.2) (layer F.Cu) (width 0.3))
  (fp_line (start -10.5 3.25) (end 10.5 3.25) (layer F.Cu) (width 0.3))
  (fp_line (start -10.5 -3.25) (end 10.5 -3.25) (layer F.Cu) (width 0.3))
  (fp_circle (center 0 0) (end 0 12.5) (layer F.SilkS) (width 0.15))
  (fp_line (start 12 -3) (end 11.5 -3) (layer F.SilkS) (width 0.15))
  (fp_line (start 12 3) (end 12 -3) (layer F.SilkS) (width 0.15))
  (fp_line (start 11.5 3) (end 12 3) (layer F.SilkS) (width 0.15))
  (fp_line (start 9 3) (end 9.5 3) (layer F.SilkS) (width 0.15))
  (fp_line (start 9 -3) (end 9 3) (layer F.SilkS) (width 0.15))
  (fp_line (start 9.5 -3) (end 9 -3) (layer F.SilkS) (width 0.15))
  (fp_line (start -11.5 -3) (end -12 -3) (layer F.SilkS) (width 0.15))
  (fp_line (start -12 -3) (end -12 3) (layer F.SilkS) (width 0.15))
  (fp_line (start -12 3) (end -11.5 3) (layer F.SilkS) (width 0.15))
  (fp_line (start -9.5 3) (end -9 3) (layer F.SilkS) (width 0.15))
  (fp_line (start -9 3) (end -9 -3) (layer F.SilkS) (width 0.15))
  (fp_line (start -9 -3) (end -9.5 -3) (layer F.SilkS) (width 0.15))
  (fp_line (start -7.5 5.2) (end -7.5 5.9) (layer F.SilkS) (width 0.15))
  (fp_line (start -7.5 5.9) (end -7.5 6.6) (layer F.SilkS) (width 0.15))
  (fp_line (start -7.5 4.4) (end -7.5 1) (layer F.SilkS) (width 0.15))
  (fp_line (start -7.5 5.2) (end -8.2 4.4) (layer F.SilkS) (width 0.15))
  (fp_line (start -8.2 4.4) (end -6.8 4.4) (layer F.SilkS) (width 0.15))
  (fp_line (start -6.8 4.4) (end -7.5 5.2) (layer F.SilkS) (width 0.15))
  (fp_line (start -8.6 5.2) (end -6.4 5.2) (layer F.SilkS) (width 0.15))
  (fp_line (start -8.6 5.9) (end -8.6 1.7) (layer F.SilkS) (width 0.15))
  (fp_line (start -8.6 1.7) (end -6.4 1.7) (layer F.SilkS) (width 0.15))
  (fp_line (start -6.4 1.7) (end -6.4 5.9) (layer F.SilkS) (width 0.15))
  (fp_line (start -6.4 5.9) (end -8.6 5.9) (layer F.SilkS) (width 0.15))
  (fp_circle (center 0 0) (end 1 1.5) (layer F.SilkS) (width 0.15))
  (fp_line (start -2.5 0) (end -2.5 -2.5) (layer F.SilkS) (width 0.15))
  (fp_line (start -2.5 -2.5) (end 2.5 -2.5) (layer F.SilkS) (width 0.15))
  (fp_line (start 2.5 -2.5) (end 2.5 2.5) (layer F.SilkS) (width 0.15))
  (fp_line (start 2.5 2.5) (end -2.5 2.5) (layer F.SilkS) (width 0.15))
  (fp_line (start -2.5 2.5) (end -2.5 0) (layer F.SilkS) (width 0.15))
  (fp_line (start -6 0) (end -6 -8.5) (layer F.SilkS) (width 0.15))
  (fp_line (start -6 -8.5) (end 6 -8.5) (layer F.SilkS) (width 0.15))
  (fp_line (start 6 -8.5) (end 6 8.5) (layer F.SilkS) (width 0.15))
  (fp_line (start 6 8.5) (end -6 8.5) (layer F.SilkS) (width 0.15))
  (fp_line (start -6 8.6) (end -6 0.1) (layer F.SilkS) (width 0.15))
  (pad 10 thru_hole circle (at 13 -3.25) (size 1 1) (drill 0.5) (layers *.Cu *.Mask) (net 3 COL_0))
  (pad "" thru_hole circle (at 10.5 -3.25) (size 2 2) (drill 1.1) (layers *.Cu *.Mask))
  (pad "" thru_hole circle (at 10.5 3.25) (size 2 2) (drill 1.1) (layers *.Cu *.Mask))
  (pad "" thru_hole circle (at -10.5 3.25) (size 2 2) (drill 1.1) (layers *.Cu *.Mask))
  (pad "" thru_hole circle (at -10.5 -3.25) (size 2 2) (drill 1.1) (layers *.Cu *.Mask))
  (pad 9 thru_hole oval (at -7.5 -0.02 90) (size 1.6 1.6) (drill 0.8) (layers *.Cu *.Mask) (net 2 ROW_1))
  (pad 5 smd rect (at -3.725 8.5) (size 1.75 4) (layers F.Cu F.Paste F.Mask) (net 22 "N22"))
  (pad 8 smd rect (at 3.925 8.5) (size 1.75 4) (layers F.Cu F.Paste F.Mask) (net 21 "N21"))
  (pad 6 smd rect (at -1.175 8.5) (size 1.75 4) (layers F.Cu F.Paste F.Mask) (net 24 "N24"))
  (pad 7 smd rect (at 1.375 8.5) (size 1.75 4) (layers F.Cu F.Paste F.Mask) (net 23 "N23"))
  (pad 3 smd rect (at 1.375 -8.5) (size 1.75 4) (layers F.Cu F.Paste F.Mask) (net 12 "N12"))
  (pad 2 smd rect (at -1.175 -8.5) (size 1.75 4) (layers F.Cu F.Paste F.Mask) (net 11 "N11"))
  (pad 4 smd rect (at 3.925 -8.5) (size 1.75 4) (layers F.Cu F.Paste F.Mask) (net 10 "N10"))
  (pad 1 smd rect (at -3.725 -8.5) (size 1.75 4) (layers F.Cu F.Paste F.Mask) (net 9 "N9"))
  (pad "" thru_hole rect (at -7.5 7.6 90) (size 1.6 1.6) (drill 0.8) (layers *.Cu *.Mask)))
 (gr_line (start 83 83) (end 145 83) (angle 90) (layer Edge.Cuts) (width 0.15))
 (gr_line (start 83 146) (end 83 83) (angle 90) (layer Edge.Cuts) (width 0.15))
 (gr_line (start 145 146) (end 145 83) (angle 90) (layer Edge.Cuts) (width 0.15))
 (gr_line (start 83 146) (end 145 146) (angle 90) (layer Edge.Cuts) (width 0.15))
 (segment (start 99.18 88.6) (end 104.85 88.6) (width 0.25) (layer B.Cu) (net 3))
 (segment (start 104.85 88.6) (end 113 96.75) (width 0.25) (layer B.Cu) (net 3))
 (segment (start 96.08 85.5) (end 99.18 88.6) (width 0.25) (layer B.Cu) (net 3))
 (segment (start 113 124.75) (end 111.924999 123.674999) (width 0.25) (layer B.Cu) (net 3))
 (segment (start 112.500001 97.249999) (end 113 96.75) (width 0.25) (layer B.Cu) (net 3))
 (segment (start 111.924999 123.674999) (end 111.924999 97.825001) (width 0.25) (layer B.Cu) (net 3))
 (segment (start 111.924999 97.825001) (end 112.500001 97.249999) (width 0.25) (layer B.Cu) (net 3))
 (segment (start 92.5 99.98) (end 120.5 99.98) (width 0.25) (layer F.Cu) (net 1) (status C00000))
 (segment (start 92.5 99.98) (end 91 98.48) (width 0.25) (layer B.Cu) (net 1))
 (segment (start 91 98.48) (end 91 85.5) (width 0.25) (layer B.Cu) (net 1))
 (segment (start 96.275 108.5) (end 96.275 119.5) (width 0.5) (layer F.Cu) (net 9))
 (segment (start 103.925 119.5) (end 103.925 108.5) (width 0.5) (layer F.Cu) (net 10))
 (segment (start 98.825 119.5) (end 98.825 108.5) (width 0.5) (layer F.Cu) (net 11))
 (segment (start 101.375 108.5) (end 101.375 119.5) (width 0.5) (layer F.Cu) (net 12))
 (segment (start 106.24 85.5) (end 106.24 86.26) (width 0.5) (layer F.Cu) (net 7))
 (segment (start 106.24 86.26) (end 104 88.5) (width 0.5) (layer F.Cu) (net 7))
 (segment (start 104 88.5) (end 102 88.5) (width 0.5) (layer F.Cu) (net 7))
 (segment (start 102 88.5) (end 101.375 89.125) (width 0.5) (layer F.Cu) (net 7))
 (segment (start 101.375 89.125) (end 101.375 91.5) (width 0.5) (layer F.Cu) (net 7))
 (segment (start 103.7 85.5) (end 103.7 86.8) (width 0.5) (layer F.Cu) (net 6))
 (segment (start 98.825 88.675) (end 98.825 91.5) (width 0.5) (layer F.Cu) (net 6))
 (segment (start 100 87.5) (end 98.825 88.675) (width 0.5) (layer F.Cu) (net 6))
 (segment (start 103 87.5) (end 100 87.5) (width 0.5) (layer F.Cu) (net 6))
 (segment (start 103.7 86.8) (end 103 87.5) (width 0.5) (layer F.Cu) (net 6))
 (segment (start 108.78 85.5) (end 108.78 86.645) (width 0.5) (layer F.Cu) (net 8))
 (segment (start 108.78 86.645) (end 103.925 91.5) (width 0.5) (layer F.Cu) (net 8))
 (segment (start 101.16 85.5) (end 100.5 85.5) (width 0.5) (layer F.Cu) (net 5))
 (segment (start 100.5 85.5) (end 96.275 89.725) (width 0.5) (layer F.Cu) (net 5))
 (segment (start 96.275 89.725) (end 96.275 91.5) (width 0.5) (layer F.Cu) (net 5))
 (segment (start 120.5 127.98) (end 92.5 127.98) (width 0.25) (layer F.Cu) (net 2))
 (segment (start 92.5 127.98) (end 92.5 125.788998) (width 0.25) (layer B.Cu) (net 2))
 (segment (start 92.5 125.788998) (end 88.174999 121.463997) (width 0.25) (layer B.Cu) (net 2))
 (segment (start 88.174999 121.463997) (end 88.174999 86.039999) (width 0.25) (layer B.Cu) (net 2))
 (segment (start 88.174999 86.039999) (end 89.889999 84.324999) (width 0.25) (layer B.Cu) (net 2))
 (segment (start 92.364999 84.324999) (end 92.690001 84.650001) (width 0.25) (layer B.Cu) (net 2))
 (segment (start 89.889999 84.324999) (end 92.364999 84.324999) (width 0.25) (layer B.Cu) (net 2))
 (segment (start 92.690001 84.650001) (end 93.54 85.5) (width 0.25) (layer B.Cu) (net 2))
 (segment (start 129.09999 141.90001) (end 131.925 139.075) (width 0.5) (layer F.Cu) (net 22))
 (segment (start 99.075 141.8) (end 109.010038 141.8) (width 0.5) (layer F.Cu) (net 22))
 (segment (start 96.275 139) (end 99.075 141.8) (width 0.5) (layer F.Cu) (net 22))
 (segment (start 96.275 136.5) (end 96.275 139) (width 0.5) (layer F.Cu) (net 22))
 (segment (start 112.310047 145.10001) (end 115.489952 145.10001) (width 0.5) (layer F.Cu) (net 22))
 (segment (start 109.010038 141.8) (end 112.310047 145.10001) (width 0.5) (layer F.Cu) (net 22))
 (segment (start 118.689952 141.90001) (end 129.09999 141.90001) (width 0.5) (layer F.Cu) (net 22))
 (segment (start 115.489952 145.10001) (end 118.689952 141.90001) (width 0.5) (layer F.Cu) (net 22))
 (segment (start 131.925 139.075) (end 131.925 136.5) (width 0.5) (layer F.Cu) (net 22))
 (segment (start 103.925 136.5) (end 103.925 137.425) (width 0.5) (layer F.Cu) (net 21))
 (segment (start 103.925 137.425) (end 105 138.5) (width 0.5) (layer F.Cu) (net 21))
 (segment (start 105 138.5) (end 122.275 138.5) (width 0.5) (layer F.Cu) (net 21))
 (segment (start 122.275 138.5) (end 124.275 136.5) (width 0.5) (layer F.Cu) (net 21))
 (segment (start 129.375 136.5) (end 129.375 138.625) (width 0.5) (layer F.Cu) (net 24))
 (segment (start 129.375 138.625) (end 126.8 141.2) (width 0.5) (layer F.Cu) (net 24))
 (segment (start 126.8 141.2) (end 118.4 141.2) (width 0.5) (layer F.Cu) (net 24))
 (segment (start 118.4 141.2) (end 115.2 144.4) (width 0.5) (layer F.Cu) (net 24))
 (segment (start 115.2 144.4) (end 112.6 144.4) (width 0.5) (layer F.Cu) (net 24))
 (segment (start 112.6 144.4) (end 109.2 141) (width 0.5) (layer F.Cu) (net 24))
 (segment (start 109.2 141) (end 100.6 141) (width 0.5) (layer F.Cu) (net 24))
 (segment (start 100.6 141) (end 98.825 139.225) (width 0.5) (layer F.Cu) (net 24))
 (segment (start 98.825 139.225) (end 98.825 136.5) (width 0.5) (layer F.Cu) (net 24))
 (segment (start 101.375 136.5) (end 101.375 137.875) (width 0.5) (layer F.Cu) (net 23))
 (segment (start 101.375 137.875) (end 103 139.5) (width 0.5) (layer F.Cu) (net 23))
 (segment (start 103 139.5) (end 126.5 139.5) (width 0.5) (layer F.Cu) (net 23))
 (segment (start 126.5 139.5) (end 126.825 139.175) (width 0.5) (layer F.Cu) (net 23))
 (segment (start 126.825 139.175) (end 126.825 136.5) (width 0.5) (layer F.Cu) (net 23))
 (segment (start 141 96.75) (end 139.924999 97.825001) (width 0.25) (layer B.Cu) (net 4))
 (segment (start 139.924999 97.825001) (end 139.924999 123.674999) (width 0.25) (layer B.Cu) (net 4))
 (segment (start 139.924999 123.674999) (end 140.500001 124.250001) (width 0.25) (layer B.Cu) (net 4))
 (segment (start 140.500001 124.250001) (end 141 124.75) (width 0.25) (layer B.Cu) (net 4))
 (segment (start 98.62 85.5) (end 101.195001 88.075001) (width 0.25) (layer B.Cu) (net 4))
 (segment (start 101.195001 88.075001) (end 132.325001 88.075001) (width 0.25) (layer B.Cu) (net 4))
 (segment (start 132.325001 88.075001) (end 140.500001 96.250001) (width 0.25) (layer B.Cu) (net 4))
 (segment (start 140.500001 96.250001) (end 141 96.75) (width 0.25) (layer B.Cu) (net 4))
 (segment (start 140.6 96.35) (end 141 96.75) (width 0.25) (layer F.Cu) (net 4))
 (segment (start 129.375 108.5) (end 129.375 119.5) (width 0.5) (layer F.Cu) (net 16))
 (segment (start 126.825 119.5) (end 126.825 108.5) (width 0.5) (layer F.Cu) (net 15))
 (segment (start 131.925 119.5) (end 131.925 108.5) (width 0.5) (layer F.Cu) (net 14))
 (segment (start 124.275 108.5) (end 124.275 119.5) (width 0.5) (layer F.Cu) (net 13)))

